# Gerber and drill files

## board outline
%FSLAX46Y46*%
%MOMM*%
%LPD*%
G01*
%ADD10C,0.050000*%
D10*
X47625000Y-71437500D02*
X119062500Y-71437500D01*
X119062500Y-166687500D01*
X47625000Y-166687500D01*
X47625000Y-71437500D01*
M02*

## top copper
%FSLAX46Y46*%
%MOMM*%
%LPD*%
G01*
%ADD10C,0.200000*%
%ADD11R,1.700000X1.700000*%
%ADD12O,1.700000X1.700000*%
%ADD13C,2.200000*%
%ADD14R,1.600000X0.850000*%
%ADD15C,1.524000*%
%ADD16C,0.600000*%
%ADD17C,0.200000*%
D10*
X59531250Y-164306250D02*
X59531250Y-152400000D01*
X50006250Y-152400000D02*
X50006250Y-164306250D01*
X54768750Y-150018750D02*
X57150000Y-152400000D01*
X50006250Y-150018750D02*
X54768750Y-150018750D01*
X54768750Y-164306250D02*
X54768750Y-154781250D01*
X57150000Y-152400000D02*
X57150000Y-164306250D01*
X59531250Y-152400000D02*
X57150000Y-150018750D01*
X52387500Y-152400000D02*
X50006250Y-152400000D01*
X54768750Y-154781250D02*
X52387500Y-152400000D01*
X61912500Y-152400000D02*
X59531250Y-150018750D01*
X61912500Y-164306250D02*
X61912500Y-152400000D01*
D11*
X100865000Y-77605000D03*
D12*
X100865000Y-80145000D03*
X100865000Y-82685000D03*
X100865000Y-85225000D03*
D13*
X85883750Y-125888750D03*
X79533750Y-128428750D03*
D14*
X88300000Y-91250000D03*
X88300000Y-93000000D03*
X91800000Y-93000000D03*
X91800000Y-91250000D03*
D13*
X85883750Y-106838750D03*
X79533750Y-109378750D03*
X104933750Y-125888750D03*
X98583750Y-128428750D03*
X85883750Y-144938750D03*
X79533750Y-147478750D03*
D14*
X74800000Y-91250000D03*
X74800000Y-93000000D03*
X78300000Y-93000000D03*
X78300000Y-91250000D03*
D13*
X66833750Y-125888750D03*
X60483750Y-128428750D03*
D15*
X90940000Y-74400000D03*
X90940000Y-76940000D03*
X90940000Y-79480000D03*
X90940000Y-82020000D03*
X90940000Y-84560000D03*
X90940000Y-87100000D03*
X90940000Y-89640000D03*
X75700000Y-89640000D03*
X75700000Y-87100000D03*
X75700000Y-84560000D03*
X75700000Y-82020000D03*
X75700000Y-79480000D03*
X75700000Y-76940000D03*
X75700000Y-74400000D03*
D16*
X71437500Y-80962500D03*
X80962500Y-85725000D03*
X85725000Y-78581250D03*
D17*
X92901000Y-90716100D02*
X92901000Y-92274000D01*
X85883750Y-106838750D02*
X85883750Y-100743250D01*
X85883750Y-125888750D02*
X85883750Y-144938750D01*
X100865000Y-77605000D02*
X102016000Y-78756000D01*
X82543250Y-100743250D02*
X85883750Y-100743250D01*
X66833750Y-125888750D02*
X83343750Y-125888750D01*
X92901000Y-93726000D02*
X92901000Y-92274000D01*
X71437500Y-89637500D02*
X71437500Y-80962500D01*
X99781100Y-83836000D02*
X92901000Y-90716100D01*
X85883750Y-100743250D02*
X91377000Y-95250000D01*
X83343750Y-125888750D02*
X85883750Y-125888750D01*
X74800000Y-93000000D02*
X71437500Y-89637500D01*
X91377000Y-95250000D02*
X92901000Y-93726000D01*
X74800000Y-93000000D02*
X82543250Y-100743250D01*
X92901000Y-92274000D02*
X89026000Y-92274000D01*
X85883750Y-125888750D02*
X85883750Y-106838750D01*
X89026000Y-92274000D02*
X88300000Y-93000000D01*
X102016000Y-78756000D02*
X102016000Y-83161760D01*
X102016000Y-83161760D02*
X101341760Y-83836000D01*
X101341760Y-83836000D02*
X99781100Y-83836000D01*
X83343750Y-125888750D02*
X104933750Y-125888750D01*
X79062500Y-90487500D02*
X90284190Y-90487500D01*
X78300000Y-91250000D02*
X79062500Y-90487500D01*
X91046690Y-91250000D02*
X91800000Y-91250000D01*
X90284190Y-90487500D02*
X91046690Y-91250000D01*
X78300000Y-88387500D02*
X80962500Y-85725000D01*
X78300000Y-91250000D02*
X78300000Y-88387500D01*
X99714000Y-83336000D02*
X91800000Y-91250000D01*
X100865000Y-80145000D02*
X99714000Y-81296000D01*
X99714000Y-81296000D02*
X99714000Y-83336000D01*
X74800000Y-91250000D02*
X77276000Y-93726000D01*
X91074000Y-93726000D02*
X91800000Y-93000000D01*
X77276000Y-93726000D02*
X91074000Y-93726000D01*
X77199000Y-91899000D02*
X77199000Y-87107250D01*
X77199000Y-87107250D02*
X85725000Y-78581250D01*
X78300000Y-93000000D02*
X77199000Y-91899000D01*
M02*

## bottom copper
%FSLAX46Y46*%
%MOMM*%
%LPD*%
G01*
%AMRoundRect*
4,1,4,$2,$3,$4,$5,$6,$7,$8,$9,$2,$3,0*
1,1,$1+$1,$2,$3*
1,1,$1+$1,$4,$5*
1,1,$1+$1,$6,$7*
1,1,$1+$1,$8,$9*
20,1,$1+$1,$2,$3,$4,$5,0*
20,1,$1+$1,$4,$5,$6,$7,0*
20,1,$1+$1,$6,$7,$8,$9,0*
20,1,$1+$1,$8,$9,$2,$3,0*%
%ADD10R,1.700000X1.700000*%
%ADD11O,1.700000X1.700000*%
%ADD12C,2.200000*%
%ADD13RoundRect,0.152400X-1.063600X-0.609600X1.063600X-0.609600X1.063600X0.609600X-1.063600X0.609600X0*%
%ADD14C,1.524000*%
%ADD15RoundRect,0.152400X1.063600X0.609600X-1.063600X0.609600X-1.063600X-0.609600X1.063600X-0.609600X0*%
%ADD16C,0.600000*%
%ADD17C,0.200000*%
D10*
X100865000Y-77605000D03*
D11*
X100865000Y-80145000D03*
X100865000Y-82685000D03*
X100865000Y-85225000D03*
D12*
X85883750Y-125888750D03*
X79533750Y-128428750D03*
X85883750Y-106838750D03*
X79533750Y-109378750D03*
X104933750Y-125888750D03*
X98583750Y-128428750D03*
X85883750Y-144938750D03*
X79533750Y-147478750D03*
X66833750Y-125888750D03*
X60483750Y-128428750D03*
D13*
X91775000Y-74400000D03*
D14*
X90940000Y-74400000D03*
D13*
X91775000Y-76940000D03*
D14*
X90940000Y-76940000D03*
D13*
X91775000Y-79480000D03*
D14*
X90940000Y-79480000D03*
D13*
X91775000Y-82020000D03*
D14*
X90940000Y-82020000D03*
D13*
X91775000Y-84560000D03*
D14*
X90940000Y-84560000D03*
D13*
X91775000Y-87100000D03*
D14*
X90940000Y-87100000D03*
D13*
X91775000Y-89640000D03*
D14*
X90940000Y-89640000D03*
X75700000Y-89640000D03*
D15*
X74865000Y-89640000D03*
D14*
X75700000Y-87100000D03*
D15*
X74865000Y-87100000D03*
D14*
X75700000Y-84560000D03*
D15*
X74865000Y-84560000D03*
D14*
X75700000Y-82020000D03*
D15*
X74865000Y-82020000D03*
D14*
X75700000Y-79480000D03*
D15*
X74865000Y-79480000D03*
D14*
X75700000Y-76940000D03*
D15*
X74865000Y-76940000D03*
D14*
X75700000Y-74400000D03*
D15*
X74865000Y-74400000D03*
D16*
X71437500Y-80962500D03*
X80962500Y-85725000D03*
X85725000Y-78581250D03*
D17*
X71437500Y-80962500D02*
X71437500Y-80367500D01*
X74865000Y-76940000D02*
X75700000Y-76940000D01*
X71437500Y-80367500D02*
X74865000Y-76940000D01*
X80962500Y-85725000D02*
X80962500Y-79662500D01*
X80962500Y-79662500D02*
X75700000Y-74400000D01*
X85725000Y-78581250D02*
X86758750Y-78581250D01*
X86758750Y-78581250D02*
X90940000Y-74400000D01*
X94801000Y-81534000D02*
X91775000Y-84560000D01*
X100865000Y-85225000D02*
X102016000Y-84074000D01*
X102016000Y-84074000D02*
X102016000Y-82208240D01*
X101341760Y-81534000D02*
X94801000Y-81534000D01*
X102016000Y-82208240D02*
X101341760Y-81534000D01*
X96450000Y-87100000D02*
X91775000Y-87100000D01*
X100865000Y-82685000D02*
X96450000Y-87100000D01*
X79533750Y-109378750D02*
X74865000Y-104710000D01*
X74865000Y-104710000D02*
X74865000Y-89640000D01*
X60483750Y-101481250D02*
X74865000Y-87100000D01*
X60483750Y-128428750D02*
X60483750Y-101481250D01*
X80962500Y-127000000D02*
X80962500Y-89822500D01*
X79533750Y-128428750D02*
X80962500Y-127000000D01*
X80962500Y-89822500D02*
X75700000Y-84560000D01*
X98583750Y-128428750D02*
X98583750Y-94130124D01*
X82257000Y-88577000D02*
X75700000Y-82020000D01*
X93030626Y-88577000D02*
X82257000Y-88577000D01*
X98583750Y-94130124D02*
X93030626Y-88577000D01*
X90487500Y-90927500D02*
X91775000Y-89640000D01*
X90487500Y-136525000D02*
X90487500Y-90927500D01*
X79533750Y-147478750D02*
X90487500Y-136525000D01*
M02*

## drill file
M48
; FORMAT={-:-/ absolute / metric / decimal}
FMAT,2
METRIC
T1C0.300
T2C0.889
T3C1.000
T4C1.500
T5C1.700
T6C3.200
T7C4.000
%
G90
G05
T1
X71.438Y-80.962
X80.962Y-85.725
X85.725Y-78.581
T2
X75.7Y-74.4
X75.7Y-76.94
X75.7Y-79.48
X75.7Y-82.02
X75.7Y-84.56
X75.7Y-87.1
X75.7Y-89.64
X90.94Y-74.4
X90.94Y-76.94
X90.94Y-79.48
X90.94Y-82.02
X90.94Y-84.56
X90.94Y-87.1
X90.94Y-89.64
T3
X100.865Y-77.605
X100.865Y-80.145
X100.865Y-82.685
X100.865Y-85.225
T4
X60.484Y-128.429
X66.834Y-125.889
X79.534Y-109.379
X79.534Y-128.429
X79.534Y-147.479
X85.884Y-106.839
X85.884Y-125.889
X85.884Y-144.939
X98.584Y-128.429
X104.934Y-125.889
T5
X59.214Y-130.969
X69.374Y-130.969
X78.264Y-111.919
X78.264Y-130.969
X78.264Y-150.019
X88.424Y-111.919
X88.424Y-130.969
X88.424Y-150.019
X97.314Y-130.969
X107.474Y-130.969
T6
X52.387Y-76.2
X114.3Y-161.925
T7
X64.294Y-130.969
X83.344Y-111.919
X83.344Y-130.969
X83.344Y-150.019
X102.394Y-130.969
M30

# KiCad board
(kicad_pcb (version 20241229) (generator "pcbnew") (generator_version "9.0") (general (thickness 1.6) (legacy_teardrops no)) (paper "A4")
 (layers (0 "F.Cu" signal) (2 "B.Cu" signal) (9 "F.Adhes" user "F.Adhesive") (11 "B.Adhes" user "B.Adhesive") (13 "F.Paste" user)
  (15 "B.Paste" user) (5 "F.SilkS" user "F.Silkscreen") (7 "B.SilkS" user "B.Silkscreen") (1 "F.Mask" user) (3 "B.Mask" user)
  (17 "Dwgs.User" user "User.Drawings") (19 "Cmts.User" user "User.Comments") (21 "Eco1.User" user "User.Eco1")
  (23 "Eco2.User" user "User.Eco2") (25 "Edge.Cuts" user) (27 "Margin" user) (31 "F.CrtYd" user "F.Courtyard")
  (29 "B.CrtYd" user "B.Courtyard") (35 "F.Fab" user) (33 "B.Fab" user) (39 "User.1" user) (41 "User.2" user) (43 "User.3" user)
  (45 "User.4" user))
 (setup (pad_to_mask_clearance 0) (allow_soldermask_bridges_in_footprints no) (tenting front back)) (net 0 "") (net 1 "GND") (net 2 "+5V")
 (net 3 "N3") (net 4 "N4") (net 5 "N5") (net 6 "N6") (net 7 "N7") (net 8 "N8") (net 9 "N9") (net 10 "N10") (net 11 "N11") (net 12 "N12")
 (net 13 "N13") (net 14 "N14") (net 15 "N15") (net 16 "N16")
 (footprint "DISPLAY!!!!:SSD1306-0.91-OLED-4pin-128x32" (layer "F.Cu") (at 64.365 75.415)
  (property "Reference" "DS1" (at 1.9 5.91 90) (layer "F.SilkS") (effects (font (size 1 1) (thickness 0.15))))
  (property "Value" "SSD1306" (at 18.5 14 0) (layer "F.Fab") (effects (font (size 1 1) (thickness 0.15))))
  (pad "1" thru_hole rect (at 36.5 2.19) (size 1.7 1.7) (drill 1) (layers "*.Cu" "*.Mask") (remove_unused_layers no) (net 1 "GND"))
  (pad "2" thru_hole oval (at 36.5 4.73) (size 1.7 1.7) (drill 1) (layers "*.Cu" "*.Mask") (remove_unused_layers no) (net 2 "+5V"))
  (pad "3" thru_hole oval (at 36.5 7.27) (size 1.7 1.7) (drill 1) (layers "*.Cu" "*.Mask") (remove_unused_layers no) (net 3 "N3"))
  (pad "4" thru_hole oval (at 36.5 9.81) (size 1.7 1.7) (drill 1) (layers "*.Cu" "*.Mask") (remove_unused_layers no) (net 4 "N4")))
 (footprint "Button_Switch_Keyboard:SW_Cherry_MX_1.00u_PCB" (layer "F.Cu") (at 85.88375 125.88875)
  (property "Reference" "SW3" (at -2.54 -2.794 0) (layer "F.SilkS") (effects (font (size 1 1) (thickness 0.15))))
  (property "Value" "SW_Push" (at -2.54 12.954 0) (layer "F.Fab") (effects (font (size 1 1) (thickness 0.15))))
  (pad "" np_thru_hole circle (at -7.62 5.08) (size 1.7 1.7) (drill 1.7) (layers "*.Cu" "*.Mask"))
  (pad "" np_thru_hole circle (at -2.54 5.08) (size 4 4) (drill 4) (layers "*.Cu" "*.Mask"))
  (pad "" np_thru_hole circle (at 2.54 5.08) (size 1.7 1.7) (drill 1.7) (layers "*.Cu" "*.Mask"))
  (pad "1" thru_hole circle (at 0 0) (size 2.2 2.2) (drill 1.5) (layers "*.Cu" "*.Mask") (remove_unused_layers no) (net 1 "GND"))
  (pad "2" thru_hole circle (at -6.35 2.54) (size 2.2 2.2) (drill 1.5) (layers "*.Cu" "*.Mask") (remove_unused_layers no) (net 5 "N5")))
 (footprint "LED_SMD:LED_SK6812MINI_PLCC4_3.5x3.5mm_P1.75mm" (layer "F.Cu") (at 90.05 92.125)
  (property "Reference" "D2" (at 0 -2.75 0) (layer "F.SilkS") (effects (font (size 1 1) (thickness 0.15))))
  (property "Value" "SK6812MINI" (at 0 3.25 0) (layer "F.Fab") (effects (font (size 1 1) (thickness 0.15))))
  (pad "1" smd rect (at -1.75 -0.875) (size 1.6 0.85) (layers "F.Cu" "F.Mask" "F.Paste") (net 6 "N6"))
  (pad "2" smd rect (at -1.75 0.875) (size 1.6 0.85) (layers "F.Cu" "F.Mask" "F.Paste") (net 1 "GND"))
  (pad "3" smd rect (at 1.75 0.875) (size 1.6 0.85) (layers "F.Cu" "F.Mask" "F.Paste") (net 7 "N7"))
  (pad "4" smd rect (at 1.75 -0.875) (size 1.6 0.85) (layers "F.Cu" "F.Mask" "F.Paste") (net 2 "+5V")))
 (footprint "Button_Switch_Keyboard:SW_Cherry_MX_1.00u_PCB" (layer "F.Cu") (at 85.88375 106.83875)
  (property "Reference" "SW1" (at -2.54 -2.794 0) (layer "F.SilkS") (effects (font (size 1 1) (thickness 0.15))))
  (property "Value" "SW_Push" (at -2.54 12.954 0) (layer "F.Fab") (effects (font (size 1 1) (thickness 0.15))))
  (pad "" np_thru_hole circle (at -7.62 5.08) (size 1.7 1.7) (drill 1.7) (layers "*.Cu" "*.Mask"))
  (pad "" np_thru_hole circle (at -2.54 5.08) (size 4 4) (drill 4) (layers "*.Cu" "*.Mask"))
  (pad "" np_thru_hole circle (at 2.54 5.08) (size 1.7 1.7) (drill 1.7) (layers "*.Cu" "*.Mask"))
  (pad "1" thru_hole circle (at 0 0) (size 2.2 2.2) (drill 1.5) (layers "*.Cu" "*.Mask") (remove_unused_layers no) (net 1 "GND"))
  (pad "2" thru_hole circle (at -6.35 2.54) (size 2.2 2.2) (drill 1.5) (layers "*.Cu" "*.Mask") (remove_unused_layers no) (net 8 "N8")))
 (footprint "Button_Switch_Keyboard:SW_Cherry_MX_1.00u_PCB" (layer "F.Cu") (at 104.93375 125.88875)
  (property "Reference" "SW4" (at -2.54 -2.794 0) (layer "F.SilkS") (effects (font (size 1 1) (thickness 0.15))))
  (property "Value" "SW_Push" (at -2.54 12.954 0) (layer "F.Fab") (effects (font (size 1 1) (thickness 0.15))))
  (pad "" np_thru_hole circle (at -7.62 5.08) (size 1.7 1.7) (drill 1.7) (layers "*.Cu" "*.Mask"))
  (pad "" np_thru_hole circle (at -2.54 5.08) (size 4 4) (drill 4) (layers "*.Cu" "*.Mask"))
  (pad "" np_thru_hole circle (at 2.54 5.08) (size 1.7 1.7) (drill 1.7) (layers "*.Cu" "*.Mask"))
  (pad "1" thru_hole circle (at 0 0) (size 2.2 2.2) (drill 1.5) (layers "*.Cu" "*.Mask") (remove_unused_layers no) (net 1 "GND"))
  (pad "2" thru_hole circle (at -6.35 2.54) (size 2.2 2.2) (drill 1.5) (layers "*.Cu" "*.Mask") (remove_unused_layers no) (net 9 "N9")))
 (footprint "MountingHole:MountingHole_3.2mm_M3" (layer "F.Cu") (at 114.3 161.925)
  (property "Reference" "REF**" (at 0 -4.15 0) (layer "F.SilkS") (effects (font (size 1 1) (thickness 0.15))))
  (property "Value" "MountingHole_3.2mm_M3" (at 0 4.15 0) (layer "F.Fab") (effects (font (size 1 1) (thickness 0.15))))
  (pad "" np_thru_hole circle (at 0 0) (size 3.2 3.2) (drill 3.2) (layers "*.Cu" "*.Mask")))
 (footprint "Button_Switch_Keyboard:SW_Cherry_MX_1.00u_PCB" (layer "F.Cu") (at 85.88375 144.93875)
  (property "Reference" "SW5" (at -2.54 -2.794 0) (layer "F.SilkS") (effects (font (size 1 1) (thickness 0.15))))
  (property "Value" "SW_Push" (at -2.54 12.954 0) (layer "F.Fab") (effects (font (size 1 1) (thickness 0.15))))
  (pad "" np_thru_hole circle (at -7.62 5.08) (size 1.7 1.7) (drill 1.7) (layers "*.Cu" "*.Mask"))
  (pad "" np_thru_hole circle (at -2.54 5.08) (size 4 4) (drill 4) (layers "*.Cu" "*.Mask"))
  (pad "" np_thru_hole circle (at 2.54 5.08) (size 1.7 1.7) (drill 1.7) (layers "*.Cu" "*.Mask"))
  (pad "1" thru_hole circle (at 0 0) (size 2.2 2.2) (drill 1.5) (layers "*.Cu" "*.Mask") (remove_unused_layers no) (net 1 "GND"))
  (pad "2" thru_hole circle (at -6.35 2.54) (size 2.2 2.2) (drill 1.5) (layers "*.Cu" "*.Mask") (remove_unused_layers no) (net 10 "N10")))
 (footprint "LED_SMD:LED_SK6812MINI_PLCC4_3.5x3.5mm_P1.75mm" (layer "F.Cu") (at 76.55 92.125)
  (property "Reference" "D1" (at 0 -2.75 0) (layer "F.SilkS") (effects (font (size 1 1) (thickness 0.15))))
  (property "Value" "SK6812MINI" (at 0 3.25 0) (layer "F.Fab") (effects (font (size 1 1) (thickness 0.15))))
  (pad "1" smd rect (at -1.75 -0.875) (size 1.6 0.85) (layers "F.Cu" "F.Mask" "F.Paste") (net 7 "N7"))
  (pad "2" smd rect (at -1.75 0.875) (size 1.6 0.85) (layers "F.Cu" "F.Mask" "F.Paste") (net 1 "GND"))
  (pad "3" smd rect (at 1.75 0.875) (size 1.6 0.85) (layers "F.Cu" "F.Mask" "F.Paste") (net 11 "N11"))
  (pad "4" smd rect (at 1.75 -0.875) (size 1.6 0.85) (layers "F.Cu" "F.Mask" "F.Paste") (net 2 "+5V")))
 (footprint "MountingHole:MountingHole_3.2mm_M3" (layer "F.Cu") (at 52.3875 76.2)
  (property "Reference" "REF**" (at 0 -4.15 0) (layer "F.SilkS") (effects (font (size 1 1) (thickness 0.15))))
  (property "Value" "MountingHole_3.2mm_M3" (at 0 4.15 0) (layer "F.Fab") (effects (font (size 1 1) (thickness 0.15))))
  (pad "" np_thru_hole circle (at 0 0) (size 3.2 3.2) (drill 3.2) (layers "*.Cu" "*.Mask")))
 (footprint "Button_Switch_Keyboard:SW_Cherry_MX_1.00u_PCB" (layer "F.Cu") (at 66.83375 125.88875)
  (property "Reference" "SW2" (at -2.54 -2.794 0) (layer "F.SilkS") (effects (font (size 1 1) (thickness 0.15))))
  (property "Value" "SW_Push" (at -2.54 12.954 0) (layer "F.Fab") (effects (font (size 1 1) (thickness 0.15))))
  (pad "" np_thru_hole circle (at -7.62 5.08) (size 1.7 1.7) (drill 1.7) (layers "*.Cu" "*.Mask"))
  (pad "" np_thru_hole circle (at -2.54 5.08) (size 4 4) (drill 4) (layers "*.Cu" "*.Mask"))
  (pad "" np_thru_hole circle (at 2.54 5.08) (size 1.7 1.7) (drill 1.7) (layers "*.Cu" "*.Mask"))
  (pad "1" thru_hole circle (at 0 0) (size 2.2 2.2) (drill 1.5) (layers "*.Cu" "*.Mask") (remove_unused_layers no) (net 1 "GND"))
  (pad "2" thru_hole circle (at -6.35 2.54) (size 2.2 2.2) (drill 1.5) (layers "*.Cu" "*.Mask") (remove_unused_layers no) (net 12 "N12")))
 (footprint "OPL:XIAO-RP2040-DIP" (layer "B.Cu") (at 83.32 82.02 180)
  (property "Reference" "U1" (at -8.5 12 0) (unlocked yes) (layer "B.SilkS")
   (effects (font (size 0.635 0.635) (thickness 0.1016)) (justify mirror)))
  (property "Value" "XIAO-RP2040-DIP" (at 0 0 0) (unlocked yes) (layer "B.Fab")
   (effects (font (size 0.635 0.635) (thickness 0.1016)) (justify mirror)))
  (pad "1" smd roundrect (at -8.455 7.62) (size 2.432 1.524) (layers "B.Cu" "B.Mask") (roundrect_rratio 0.1) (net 11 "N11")
   (thermal_bridge_angle 45))
  (pad "1" thru_hole circle (at -7.62 7.62) (size 1.524 1.524) (drill 0.889) (layers "*.Cu" "*.Mask") (remove_unused_layers no)
   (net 11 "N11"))
  (pad "2" smd roundrect (at -8.455 5.08) (size 2.432 1.524) (layers "B.Cu" "B.Mask") (roundrect_rratio 0.1) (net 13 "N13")
   (thermal_bridge_angle 45))
  (pad "2" thru_hole circle (at -7.62 5.08) (size 1.524 1.524) (drill 0.889) (layers "*.Cu" "*.Mask") (remove_unused_layers no)
   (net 13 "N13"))
  (pad "3" smd roundrect (at -8.455 2.54) (size 2.432 1.524) (layers "B.Cu" "B.Mask") (roundrect_rratio 0.1) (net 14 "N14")
   (thermal_bridge_angle 45))
  (pad "3" thru_hole circle (at -7.62 2.54) (size 1.524 1.524) (drill 0.889) (layers "*.Cu" "*.Mask") (remove_unused_layers no)
   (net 14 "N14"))
  (pad "4" smd roundrect (at -8.455 0) (size 2.432 1.524) (layers "B.Cu" "B.Mask") (roundrect_rratio 0.1) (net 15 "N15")
   (thermal_bridge_angle 45))
  (pad "4" thru_hole circle (at -7.62 0) (size 1.524 1.524) (drill 0.889) (layers "*.Cu" "*.Mask") (remove_unused_layers no) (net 15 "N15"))
  (pad "5" smd roundrect (at -8.455 -2.54) (size 2.432 1.524) (layers "B.Cu" "B.Mask") (roundrect_rratio 0.1) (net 4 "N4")
   (thermal_bridge_angle 45))
  (pad "5" thru_hole circle (at -7.62 -2.54) (size 1.524 1.524) (drill 0.889) (layers "*.Cu" "*.Mask") (remove_unused_layers no)
   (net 4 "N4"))
  (pad "6" smd roundrect (at -8.455 -5.08) (size 2.432 1.524) (layers "B.Cu" "B.Mask") (roundrect_rratio 0.1) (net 3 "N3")
   (thermal_bridge_angle 45))
  (pad "6" thru_hole circle (at -7.62 -5.08) (size 1.524 1.524) (drill 0.889) (layers "*.Cu" "*.Mask") (remove_unused_layers no)
   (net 3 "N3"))
  (pad "7" smd roundrect (at -8.455 -7.62) (size 2.432 1.524) (layers "B.Cu" "B.Mask") (roundrect_rratio 0.1) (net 10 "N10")
   (thermal_bridge_angle 45))
  (pad "7" thru_hole circle (at -7.62 -7.62) (size 1.524 1.524) (drill 0.889) (layers "*.Cu" "*.Mask") (remove_unused_layers no)
   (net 10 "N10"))
  (pad "8" thru_hole circle (at 7.62 -7.62 180) (size 1.524 1.524) (drill 0.889) (layers "*.Cu" "*.Mask") (remove_unused_layers no)
   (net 8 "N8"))
  (pad "8" smd roundrect (at 8.455 -7.62 180) (size 2.432 1.524) (layers "B.Cu" "B.Mask") (roundrect_rratio 0.1) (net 8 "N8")
   (thermal_bridge_angle 45))
  (pad "9" thru_hole circle (at 7.62 -5.08 180) (size 1.524 1.524) (drill 0.889) (layers "*.Cu" "*.Mask") (remove_unused_layers no)
   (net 12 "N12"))
  (pad "9" smd roundrect (at 8.455 -5.08 180) (size 2.432 1.524) (layers "B.Cu" "B.Mask") (roundrect_rratio 0.1) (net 12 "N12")
   (thermal_bridge_angle 45))
  (pad "10" thru_hole circle (at 7.62 -2.54 180) (size 1.524 1.524) (drill 0.889) (layers "*.Cu" "*.Mask") (remove_unused_layers no)
   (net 5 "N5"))
  (pad "10" smd roundrect (at 8.455 -2.54 180) (size 2.432 1.524) (layers "B.Cu" "B.Mask") (roundrect_rratio 0.1) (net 5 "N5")
   (thermal_bridge_angle 45))
  (pad "11" thru_hole circle (at 7.62 0 180) (size 1.524 1.524) (drill 0.889) (layers "*.Cu" "*.Mask") (remove_unused_layers no)
   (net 9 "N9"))
  (pad "11" smd roundrect (at 8.455 0 180) (size 2.432 1.524) (layers "B.Cu" "B.Mask") (roundrect_rratio 0.1) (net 9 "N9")
   (thermal_bridge_angle 45))
  (pad "12" thru_hole circle (at 7.62 2.54 180) (size 1.524 1.524) (drill 0.889) (layers "*.Cu" "*.Mask") (remove_unused_layers no)
   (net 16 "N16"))
  (pad "12" smd roundrect (at 8.455 2.54 180) (size 2.432 1.524) (layers "B.Cu" "B.Mask") (roundrect_rratio 0.1) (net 16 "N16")
   (thermal_bridge_angle 45))
  (pad "13" thru_hole circle (at 7.62 5.08 180) (size 1.524 1.524) (drill 0.889) (layers "*.Cu" "*.Mask") (remove_unused_layers no)
   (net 1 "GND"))
  (pad "13" smd roundrect (at 8.455 5.08 180) (size 2.432 1.524) (layers "B.Cu" "B.Mask") (roundrect_rratio 0.1) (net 1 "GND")
   (thermal_bridge_angle 45))
  (pad "14" thru_hole circle (at 7.62 7.62 180) (size 1.524 1.524) (drill 0.889) (layers "*.Cu" "*.Mask") (remove_unused_layers no)
   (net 2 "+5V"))
  (pad "14" smd roundrect (at 8.455 7.62 180) (size 2.432 1.524) (layers "B.Cu" "B.Mask") (roundrect_rratio 0.1) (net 2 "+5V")
   (thermal_bridge_angle 45)))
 (gr_line (start 59.53125 164.30625) (end 59.53125 152.4) (stroke (width 0.2) (type default)) (layer "F.Cu"))
 (gr_line (start 50.00625 152.4) (end 50.00625 164.30625) (stroke (width 0.2) (type default)) (layer "F.Cu"))
 (gr_line (start 54.76875 150.01875) (end 57.15 152.4) (stroke (width 0.2) (type default)) (layer "F.Cu"))
 (gr_line (start 50.00625 150.01875) (end 54.76875 150.01875) (stroke (width 0.2) (type default)) (layer "F.Cu"))
 (gr_line (start 54.76875 164.30625) (end 54.76875 154.78125) (stroke (width 0.2) (type default)) (layer "F.Cu"))
 (gr_line (start 57.15 152.4) (end 57.15 164.30625) (stroke (width 0.2) (type default)) (layer "F.Cu"))
 (gr_line (start 59.53125 152.4) (end 57.15 150.01875) (stroke (width 0.2) (type default)) (layer "F.Cu"))
 (gr_line (start 52.3875 152.4) (end 50.00625 152.4) (stroke (width 0.2) (type default)) (layer "F.Cu"))
 (gr_line (start 54.76875 154.78125) (end 52.3875 152.4) (stroke (width 0.2) (type default)) (layer "F.Cu"))
 (gr_line (start 61.9125 152.4) (end 59.53125 150.01875) (stroke (width 0.2) (type default)) (layer "F.Cu"))
 (gr_line (start 61.9125 164.30625) (end 61.9125 152.4) (stroke (width 0.2) (type default)) (layer "F.Cu"))
 (gr_rect (start 47.625 71.4375) (end 119.0625 166.6875) (stroke (width 0.05) (type default)) (fill no) (layer "Edge.Cuts"))
 (segment (start 92.901 90.7161) (end 92.901 92.274) (width 0.2) (layer "F.Cu") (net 1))
 (segment (start 85.88375 106.83875) (end 85.88375 100.74325) (width 0.2) (layer "F.Cu") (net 1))
 (segment (start 85.88375 125.88875) (end 85.88375 144.93875) (width 0.2) (layer "F.Cu") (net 1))
 (segment (start 100.865 77.605) (end 102.016 78.756) (width 0.2) (layer "F.Cu") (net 1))
 (segment (start 82.54325 100.74325) (end 85.88375 100.74325) (width 0.2) (layer "F.Cu") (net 1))
 (segment (start 66.83375 125.88875) (end 83.34375 125.88875) (width 0.2) (layer "F.Cu") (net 1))
 (segment (start 92.901 93.726) (end 92.901 92.274) (width 0.2) (layer "F.Cu") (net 1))
 (segment (start 71.4375 89.6375) (end 71.4375 80.9625) (width 0.2) (layer "F.Cu") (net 1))
 (segment (start 99.7811 83.836) (end 92.901 90.7161) (width 0.2) (layer "F.Cu") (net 1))
 (segment (start 85.88375 100.74325) (end 91.377 95.25) (width 0.2) (layer "F.Cu") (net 1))
 (segment (start 83.34375 125.88875) (end 85.88375 125.88875) (width 0.2) (layer "F.Cu") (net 1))
 (segment (start 74.8 93) (end 71.4375 89.6375) (width 0.2) (layer "F.Cu") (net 1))
 (segment (start 91.377 95.25) (end 92.901 93.726) (width 0.2) (layer "F.Cu") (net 1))
 (segment (start 74.8 93) (end 82.54325 100.74325) (width 0.2) (layer "F.Cu") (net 1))
 (segment (start 92.901 92.274) (end 89.026 92.274) (width 0.2) (layer "F.Cu") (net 1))
 (segment (start 85.88375 125.88875) (end 85.88375 106.83875) (width 0.2) (layer "F.Cu") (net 1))
 (segment (start 89.026 92.274) (end 88.3 93) (width 0.2) (layer "F.Cu") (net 1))
 (segment (start 102.016 78.756) (end 102.016 83.16176) (width 0.2) (layer "F.Cu") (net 1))
 (segment (start 102.016 83.16176) (end 101.34176 83.836) (width 0.2) (layer "F.Cu") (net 1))
 (segment (start 101.34176 83.836) (end 99.7811 83.836) (width 0.2) (layer "F.Cu") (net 1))
 (segment (start 83.34375 125.88875) (end 104.93375 125.88875) (width 0.2) (layer "F.Cu") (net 1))
 (via (at 71.4375 80.9625) (size 0.6) (drill 0.3) (layers "F.Cu" "B.Cu") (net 1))
 (segment (start 71.4375 80.9625) (end 71.4375 80.3675) (width 0.2) (layer "B.Cu") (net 1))
 (segment (start 74.865 76.94) (end 75.7 76.94) (width 0.2) (layer "B.Cu") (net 1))
 (segment (start 71.4375 80.3675) (end 74.865 76.94) (width 0.2) (layer "B.Cu") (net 1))
 (segment (start 79.0625 90.4875) (end 90.28419 90.4875) (width 0.2) (layer "F.Cu") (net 2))
 (segment (start 78.3 91.25) (end 79.0625 90.4875) (width 0.2) (layer "F.Cu") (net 2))
 (segment (start 91.04669 91.25) (end 91.8 91.25) (width 0.2) (layer "F.Cu") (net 2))
 (segment (start 90.28419 90.4875) (end 91.04669 91.25) (width 0.2) (layer "F.Cu") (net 2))
 (segment (start 78.3 88.3875) (end 80.9625 85.725) (width 0.2) (layer "F.Cu") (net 2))
 (segment (start 78.3 91.25) (end 78.3 88.3875) (width 0.2) (layer "F.Cu") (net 2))
 (segment (start 99.714 83.336) (end 91.8 91.25) (width 0.2) (layer "F.Cu") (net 2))
 (segment (start 100.865 80.145) (end 99.714 81.296) (width 0.2) (layer "F.Cu") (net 2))
 (segment (start 99.714 81.296) (end 99.714 83.336) (width 0.2) (layer "F.Cu") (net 2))
 (via (at 80.9625 85.725) (size 0.6) (drill 0.3) (layers "F.Cu" "B.Cu") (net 2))
 (segment (start 80.9625 85.725) (end 80.9625 79.6625) (width 0.2) (layer "B.Cu") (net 2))
 (segment (start 80.9625 79.6625) (end 75.7 74.4) (width 0.2) (layer "B.Cu") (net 2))
 (segment (start 74.8 91.25) (end 77.276 93.726) (width 0.2) (layer "F.Cu") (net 7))
 (segment (start 91.074 93.726) (end 91.8 93) (width 0.2) (layer "F.Cu") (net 7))
 (segment (start 77.276 93.726) (end 91.074 93.726) (width 0.2) (layer "F.Cu") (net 7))
 (segment (start 77.199 91.899) (end 77.199 87.10725) (width 0.2) (layer "F.Cu") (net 11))
 (segment (start 77.199 87.10725) (end 85.725 78.58125) (width 0.2) (layer "F.Cu") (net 11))
 (segment (start 78.3 93) (end 77.199 91.899) (width 0.2) (layer "F.Cu") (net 11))
 (via (at 85.725 78.58125) (size 0.6) (drill 0.3) (layers "F.Cu" "B.Cu") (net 11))
 (segment (start 85.725 78.58125) (end 86.75875 78.58125) (width 0.2) (layer "B.Cu") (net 11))
 (segment (start 86.75875 78.58125) (end 90.94 74.4) (width 0.2) (layer "B.Cu") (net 11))
 (segment (start 94.801 81.534) (end 91.775 84.56) (width 0.2) (layer "B.Cu") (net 4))
 (segment (start 100.865 85.225) (end 102.016 84.074) (width 0.2) (layer "B.Cu") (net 4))
 (segment (start 102.016 84.074) (end 102.016 82.20824) (width 0.2) (layer "B.Cu") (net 4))
 (segment (start 101.34176 81.534) (end 94.801 81.534) (width 0.2) (layer "B.Cu") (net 4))
 (segment (start 102.016 82.20824) (end 101.34176 81.534) (width 0.2) (layer "B.Cu") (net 4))
 (segment (start 96.45 87.1) (end 91.775 87.1) (width 0.2) (layer "B.Cu") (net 3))
 (segment (start 100.865 82.685) (end 96.45 87.1) (width 0.2) (layer "B.Cu") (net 3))
 (segment (start 79.53375 109.37875) (end 74.865 104.71) (width 0.2) (layer "B.Cu") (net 8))
 (segment (start 74.865 104.71) (end 74.865 89.64) (width 0.2) (layer "B.Cu") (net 8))
 (segment (start 60.48375 101.48125) (end 74.865 87.1) (width 0.2) (layer "B.Cu") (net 12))
 (segment (start 60.48375 128.42875) (end 60.48375 101.48125) (width 0.2) (layer "B.Cu") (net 12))
 (segment (start 80.9625 127) (end 80.9625 89.8225) (width 0.2) (layer "B.Cu") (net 5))
 (segment (start 79.53375 128.42875) (end 80.9625 127) (width 0.2) (layer "B.Cu") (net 5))
 (segment (start 80.9625 89.8225) (end 75.7 84.56) (width 0.2) (layer "B.Cu") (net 5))
 (segment (start 98.58375 128.42875) (end 98.58375 94.130124) (width 0.2) (layer "B.Cu") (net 9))
 (segment (start 82.257 88.577) (end 75.7 82.02) (width 0.2) (layer "B.Cu") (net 9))
 (segment (start 93.030626 88.577) (end 82.257 88.577) (width 0.2) (layer "B.Cu") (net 9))
 (segment (start 98.58375 94.130124) (end 93.030626 88.577) (width 0.2) (layer "B.Cu") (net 9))
 (segment (start 90.4875 90.9275) (end 91.775 89.64) (width 0.2) (layer "B.Cu") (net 10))
 (segment (start 90.4875 136.525) (end 90.4875 90.9275) (width 0.2) (layer "B.Cu") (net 10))
 (segment (start 79.53375 147.47875) (end 90.4875 136.525) (width 0.2) (layer "B.Cu") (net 10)))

